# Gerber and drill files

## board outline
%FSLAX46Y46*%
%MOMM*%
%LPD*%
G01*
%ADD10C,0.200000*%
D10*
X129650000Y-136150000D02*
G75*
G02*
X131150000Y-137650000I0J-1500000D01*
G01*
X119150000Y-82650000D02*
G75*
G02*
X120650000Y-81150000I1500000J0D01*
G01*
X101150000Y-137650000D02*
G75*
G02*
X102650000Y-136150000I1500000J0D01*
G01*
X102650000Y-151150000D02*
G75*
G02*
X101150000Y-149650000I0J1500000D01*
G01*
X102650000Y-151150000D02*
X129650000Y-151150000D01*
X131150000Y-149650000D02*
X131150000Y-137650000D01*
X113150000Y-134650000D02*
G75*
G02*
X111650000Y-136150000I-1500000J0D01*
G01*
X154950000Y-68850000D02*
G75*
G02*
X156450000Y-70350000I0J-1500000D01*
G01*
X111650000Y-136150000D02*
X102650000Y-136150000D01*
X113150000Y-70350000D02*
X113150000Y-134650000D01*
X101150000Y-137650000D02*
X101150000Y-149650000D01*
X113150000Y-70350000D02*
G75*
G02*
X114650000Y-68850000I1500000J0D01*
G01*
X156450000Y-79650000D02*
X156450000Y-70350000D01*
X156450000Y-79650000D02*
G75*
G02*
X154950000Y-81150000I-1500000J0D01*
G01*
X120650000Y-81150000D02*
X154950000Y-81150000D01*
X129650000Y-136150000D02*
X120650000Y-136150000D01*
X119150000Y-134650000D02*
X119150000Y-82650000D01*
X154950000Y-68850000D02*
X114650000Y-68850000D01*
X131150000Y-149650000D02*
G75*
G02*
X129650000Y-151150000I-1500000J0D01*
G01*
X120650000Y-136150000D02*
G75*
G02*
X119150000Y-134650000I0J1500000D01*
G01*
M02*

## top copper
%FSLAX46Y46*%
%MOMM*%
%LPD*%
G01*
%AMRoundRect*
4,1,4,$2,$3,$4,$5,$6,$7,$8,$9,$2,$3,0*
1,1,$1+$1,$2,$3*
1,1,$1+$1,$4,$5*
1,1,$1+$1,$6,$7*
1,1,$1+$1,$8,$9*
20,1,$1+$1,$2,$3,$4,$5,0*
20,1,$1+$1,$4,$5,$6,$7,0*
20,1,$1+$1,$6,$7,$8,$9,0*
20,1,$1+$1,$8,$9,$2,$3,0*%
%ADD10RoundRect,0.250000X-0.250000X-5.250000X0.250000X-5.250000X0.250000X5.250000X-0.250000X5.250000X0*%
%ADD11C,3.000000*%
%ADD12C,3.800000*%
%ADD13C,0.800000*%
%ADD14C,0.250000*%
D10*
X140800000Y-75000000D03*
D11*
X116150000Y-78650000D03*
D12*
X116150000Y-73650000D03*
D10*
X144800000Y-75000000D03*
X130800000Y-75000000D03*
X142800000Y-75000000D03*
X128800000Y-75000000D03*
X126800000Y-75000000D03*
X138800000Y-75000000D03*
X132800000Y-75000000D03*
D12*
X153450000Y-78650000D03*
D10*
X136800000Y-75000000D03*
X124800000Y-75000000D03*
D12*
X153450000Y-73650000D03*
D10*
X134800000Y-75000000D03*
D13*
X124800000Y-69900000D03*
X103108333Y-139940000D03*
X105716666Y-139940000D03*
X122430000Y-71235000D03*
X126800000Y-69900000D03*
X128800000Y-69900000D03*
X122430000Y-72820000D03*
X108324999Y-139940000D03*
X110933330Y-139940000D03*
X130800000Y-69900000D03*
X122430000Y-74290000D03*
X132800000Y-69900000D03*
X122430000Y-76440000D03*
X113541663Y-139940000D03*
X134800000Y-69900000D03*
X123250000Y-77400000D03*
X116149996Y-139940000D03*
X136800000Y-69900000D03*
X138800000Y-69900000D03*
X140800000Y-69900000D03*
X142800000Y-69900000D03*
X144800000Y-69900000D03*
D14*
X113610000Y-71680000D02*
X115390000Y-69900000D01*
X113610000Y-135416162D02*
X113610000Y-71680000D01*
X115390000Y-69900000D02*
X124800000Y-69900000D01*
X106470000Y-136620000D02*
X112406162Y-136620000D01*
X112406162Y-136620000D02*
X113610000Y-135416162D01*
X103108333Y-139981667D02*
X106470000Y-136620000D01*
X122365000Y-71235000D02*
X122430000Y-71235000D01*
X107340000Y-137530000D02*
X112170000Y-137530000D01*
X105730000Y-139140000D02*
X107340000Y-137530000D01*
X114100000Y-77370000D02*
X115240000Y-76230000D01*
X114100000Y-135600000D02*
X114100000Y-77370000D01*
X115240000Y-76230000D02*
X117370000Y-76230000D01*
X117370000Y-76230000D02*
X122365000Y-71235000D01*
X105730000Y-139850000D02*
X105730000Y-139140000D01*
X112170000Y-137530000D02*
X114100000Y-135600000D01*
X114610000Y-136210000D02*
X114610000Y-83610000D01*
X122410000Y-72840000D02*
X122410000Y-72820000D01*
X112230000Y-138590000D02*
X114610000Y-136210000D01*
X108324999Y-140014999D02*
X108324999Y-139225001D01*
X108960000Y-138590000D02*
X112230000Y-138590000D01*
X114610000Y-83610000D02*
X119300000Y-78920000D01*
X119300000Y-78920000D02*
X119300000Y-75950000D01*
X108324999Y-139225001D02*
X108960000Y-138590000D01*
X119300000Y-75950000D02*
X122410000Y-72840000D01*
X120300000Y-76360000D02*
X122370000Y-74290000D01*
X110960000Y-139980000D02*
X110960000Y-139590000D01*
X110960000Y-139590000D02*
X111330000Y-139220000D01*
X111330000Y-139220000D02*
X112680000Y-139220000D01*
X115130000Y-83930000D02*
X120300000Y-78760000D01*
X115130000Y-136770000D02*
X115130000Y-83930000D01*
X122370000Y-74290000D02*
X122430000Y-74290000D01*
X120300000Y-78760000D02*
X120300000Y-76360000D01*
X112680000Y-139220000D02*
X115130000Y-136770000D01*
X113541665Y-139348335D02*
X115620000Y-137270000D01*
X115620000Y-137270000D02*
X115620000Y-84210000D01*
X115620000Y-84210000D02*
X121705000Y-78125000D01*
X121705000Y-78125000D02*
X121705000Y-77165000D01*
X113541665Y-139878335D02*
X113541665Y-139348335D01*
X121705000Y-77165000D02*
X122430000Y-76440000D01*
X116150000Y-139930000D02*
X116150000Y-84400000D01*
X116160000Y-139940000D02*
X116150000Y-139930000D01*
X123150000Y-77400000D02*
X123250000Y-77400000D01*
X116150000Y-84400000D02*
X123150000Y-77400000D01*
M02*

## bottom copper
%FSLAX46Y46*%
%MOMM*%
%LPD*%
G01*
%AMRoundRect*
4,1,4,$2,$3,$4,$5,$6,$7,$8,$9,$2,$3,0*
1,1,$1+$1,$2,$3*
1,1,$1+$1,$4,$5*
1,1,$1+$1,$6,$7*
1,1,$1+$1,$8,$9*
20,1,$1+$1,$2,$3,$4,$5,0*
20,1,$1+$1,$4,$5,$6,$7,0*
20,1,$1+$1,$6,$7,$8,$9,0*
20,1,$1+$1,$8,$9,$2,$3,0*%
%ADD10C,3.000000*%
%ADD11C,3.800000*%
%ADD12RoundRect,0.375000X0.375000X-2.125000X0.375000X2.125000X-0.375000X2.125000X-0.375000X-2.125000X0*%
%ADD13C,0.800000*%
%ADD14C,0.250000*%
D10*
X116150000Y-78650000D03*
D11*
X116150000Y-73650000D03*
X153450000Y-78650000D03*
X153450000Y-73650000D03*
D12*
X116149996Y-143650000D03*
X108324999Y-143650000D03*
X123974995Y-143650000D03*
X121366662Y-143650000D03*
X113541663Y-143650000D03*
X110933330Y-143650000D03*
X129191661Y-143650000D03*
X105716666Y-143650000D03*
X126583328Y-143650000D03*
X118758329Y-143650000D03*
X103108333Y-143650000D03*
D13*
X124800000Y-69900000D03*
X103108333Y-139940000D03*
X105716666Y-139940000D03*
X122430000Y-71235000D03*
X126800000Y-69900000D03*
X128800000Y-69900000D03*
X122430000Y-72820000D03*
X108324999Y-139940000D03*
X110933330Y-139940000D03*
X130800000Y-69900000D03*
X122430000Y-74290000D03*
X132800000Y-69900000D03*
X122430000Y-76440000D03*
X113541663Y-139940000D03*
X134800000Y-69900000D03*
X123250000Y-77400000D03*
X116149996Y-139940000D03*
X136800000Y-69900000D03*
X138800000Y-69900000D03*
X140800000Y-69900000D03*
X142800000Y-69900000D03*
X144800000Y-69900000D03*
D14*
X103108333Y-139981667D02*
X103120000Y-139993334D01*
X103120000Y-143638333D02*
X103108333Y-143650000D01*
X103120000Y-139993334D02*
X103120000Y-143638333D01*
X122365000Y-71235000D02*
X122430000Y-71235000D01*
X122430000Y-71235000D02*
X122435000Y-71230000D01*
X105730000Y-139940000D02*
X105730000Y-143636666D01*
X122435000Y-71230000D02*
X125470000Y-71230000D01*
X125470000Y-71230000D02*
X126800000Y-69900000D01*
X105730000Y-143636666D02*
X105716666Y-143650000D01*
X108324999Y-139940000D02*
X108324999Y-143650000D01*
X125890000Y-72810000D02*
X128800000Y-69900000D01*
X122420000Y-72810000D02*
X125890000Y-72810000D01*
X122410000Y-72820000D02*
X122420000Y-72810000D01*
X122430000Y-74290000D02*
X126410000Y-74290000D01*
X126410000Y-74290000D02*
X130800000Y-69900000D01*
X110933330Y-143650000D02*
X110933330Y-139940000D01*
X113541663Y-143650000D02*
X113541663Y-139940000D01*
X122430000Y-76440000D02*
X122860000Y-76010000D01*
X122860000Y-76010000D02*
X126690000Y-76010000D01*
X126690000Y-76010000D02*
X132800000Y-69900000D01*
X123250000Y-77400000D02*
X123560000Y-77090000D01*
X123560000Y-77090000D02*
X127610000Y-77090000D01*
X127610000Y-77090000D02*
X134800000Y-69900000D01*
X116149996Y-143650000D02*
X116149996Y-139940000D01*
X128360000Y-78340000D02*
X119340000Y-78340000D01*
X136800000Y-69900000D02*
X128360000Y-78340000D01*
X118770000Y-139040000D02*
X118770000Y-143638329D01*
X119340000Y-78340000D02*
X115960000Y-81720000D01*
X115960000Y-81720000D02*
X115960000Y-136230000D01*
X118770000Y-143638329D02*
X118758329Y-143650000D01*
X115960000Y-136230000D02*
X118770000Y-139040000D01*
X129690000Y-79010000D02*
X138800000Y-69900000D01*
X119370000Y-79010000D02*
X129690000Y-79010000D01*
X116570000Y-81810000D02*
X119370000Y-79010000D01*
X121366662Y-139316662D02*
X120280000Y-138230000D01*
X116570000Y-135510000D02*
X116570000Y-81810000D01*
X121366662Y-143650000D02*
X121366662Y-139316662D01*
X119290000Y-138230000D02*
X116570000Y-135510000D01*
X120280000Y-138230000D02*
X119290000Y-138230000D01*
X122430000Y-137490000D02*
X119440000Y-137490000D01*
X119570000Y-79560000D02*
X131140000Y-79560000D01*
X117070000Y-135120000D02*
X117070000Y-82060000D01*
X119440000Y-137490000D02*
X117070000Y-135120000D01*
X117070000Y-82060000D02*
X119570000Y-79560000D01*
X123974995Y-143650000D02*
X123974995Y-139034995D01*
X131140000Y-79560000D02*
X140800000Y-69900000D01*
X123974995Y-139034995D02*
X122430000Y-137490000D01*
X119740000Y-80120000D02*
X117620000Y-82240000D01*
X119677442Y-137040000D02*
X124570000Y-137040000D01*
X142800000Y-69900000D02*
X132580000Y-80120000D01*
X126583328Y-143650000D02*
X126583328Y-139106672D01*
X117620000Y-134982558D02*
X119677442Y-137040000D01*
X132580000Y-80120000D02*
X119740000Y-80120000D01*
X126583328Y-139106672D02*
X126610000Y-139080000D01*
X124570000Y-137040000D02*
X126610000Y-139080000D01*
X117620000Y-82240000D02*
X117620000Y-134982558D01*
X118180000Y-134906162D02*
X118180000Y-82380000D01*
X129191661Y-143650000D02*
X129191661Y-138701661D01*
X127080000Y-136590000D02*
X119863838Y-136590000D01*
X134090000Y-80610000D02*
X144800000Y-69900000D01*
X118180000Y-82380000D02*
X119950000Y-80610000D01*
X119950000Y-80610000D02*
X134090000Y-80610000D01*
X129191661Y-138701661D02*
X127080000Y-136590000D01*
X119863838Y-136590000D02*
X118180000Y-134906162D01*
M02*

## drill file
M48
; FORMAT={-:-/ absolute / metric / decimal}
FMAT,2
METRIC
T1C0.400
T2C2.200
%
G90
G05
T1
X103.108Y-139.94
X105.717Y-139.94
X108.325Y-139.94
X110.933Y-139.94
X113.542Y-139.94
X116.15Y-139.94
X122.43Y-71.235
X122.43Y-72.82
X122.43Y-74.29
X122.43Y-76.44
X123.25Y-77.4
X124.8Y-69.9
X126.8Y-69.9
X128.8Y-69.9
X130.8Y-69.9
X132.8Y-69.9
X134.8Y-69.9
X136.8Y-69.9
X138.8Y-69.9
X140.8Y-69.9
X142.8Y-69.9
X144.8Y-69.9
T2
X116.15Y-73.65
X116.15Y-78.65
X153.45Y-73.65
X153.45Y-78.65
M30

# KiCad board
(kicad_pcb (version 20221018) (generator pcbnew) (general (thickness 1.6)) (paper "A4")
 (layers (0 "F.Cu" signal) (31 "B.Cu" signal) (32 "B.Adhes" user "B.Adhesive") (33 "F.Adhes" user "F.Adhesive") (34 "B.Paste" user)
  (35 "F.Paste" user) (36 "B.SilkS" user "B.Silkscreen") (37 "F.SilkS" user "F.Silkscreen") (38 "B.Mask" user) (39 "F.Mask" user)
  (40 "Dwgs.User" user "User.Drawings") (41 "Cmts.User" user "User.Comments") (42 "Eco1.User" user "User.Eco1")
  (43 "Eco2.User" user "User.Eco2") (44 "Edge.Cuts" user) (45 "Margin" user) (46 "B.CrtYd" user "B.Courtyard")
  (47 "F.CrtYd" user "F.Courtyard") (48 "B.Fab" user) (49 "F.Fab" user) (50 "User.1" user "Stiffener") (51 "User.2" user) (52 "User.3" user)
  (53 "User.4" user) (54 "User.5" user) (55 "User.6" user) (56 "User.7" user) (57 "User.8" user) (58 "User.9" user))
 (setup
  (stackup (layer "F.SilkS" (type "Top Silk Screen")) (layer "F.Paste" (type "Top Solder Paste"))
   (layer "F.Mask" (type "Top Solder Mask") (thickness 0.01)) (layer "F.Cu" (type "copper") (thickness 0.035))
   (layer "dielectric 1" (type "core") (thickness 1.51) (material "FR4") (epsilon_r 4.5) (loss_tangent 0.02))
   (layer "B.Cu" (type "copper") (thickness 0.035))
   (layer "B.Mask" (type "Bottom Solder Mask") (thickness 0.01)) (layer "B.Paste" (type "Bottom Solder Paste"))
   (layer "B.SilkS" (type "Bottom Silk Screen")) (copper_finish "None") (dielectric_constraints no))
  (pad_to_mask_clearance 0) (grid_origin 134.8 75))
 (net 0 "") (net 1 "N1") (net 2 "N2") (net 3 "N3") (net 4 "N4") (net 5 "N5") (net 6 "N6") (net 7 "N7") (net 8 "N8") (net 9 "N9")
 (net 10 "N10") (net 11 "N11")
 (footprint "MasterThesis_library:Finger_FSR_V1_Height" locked (layer "F.Cu") (at 140.8 75)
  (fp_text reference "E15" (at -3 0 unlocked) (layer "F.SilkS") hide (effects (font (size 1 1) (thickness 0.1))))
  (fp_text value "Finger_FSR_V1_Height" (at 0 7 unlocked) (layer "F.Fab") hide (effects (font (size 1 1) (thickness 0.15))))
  (pad "1" smd roundrect locked (at 0 0) (size 1 11) (layers "F.Cu" "F.Paste" "F.Mask") (roundrect_rratio 0.25) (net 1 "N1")
   (thermal_bridge_angle 45)))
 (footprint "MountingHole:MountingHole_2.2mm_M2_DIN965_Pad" (layer "F.Cu") (at 116.15 78.65)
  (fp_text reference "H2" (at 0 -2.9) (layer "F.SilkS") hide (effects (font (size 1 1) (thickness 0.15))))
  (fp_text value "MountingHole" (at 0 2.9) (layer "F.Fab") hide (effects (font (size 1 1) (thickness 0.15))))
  (pad "1" thru_hole circle (at 0 0) (size 3 3) (drill 2.2) (layers "*.Cu" "*.Mask")))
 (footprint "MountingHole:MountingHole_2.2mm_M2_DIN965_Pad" (layer "F.Cu") (at 116.15 73.65)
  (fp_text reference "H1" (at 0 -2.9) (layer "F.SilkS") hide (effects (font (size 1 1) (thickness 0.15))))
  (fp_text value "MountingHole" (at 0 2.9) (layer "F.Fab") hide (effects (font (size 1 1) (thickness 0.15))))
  (pad "1" thru_hole circle (at 0 0) (size 3.8 3.8) (drill 2.2) (layers "*.Cu" "*.Mask")))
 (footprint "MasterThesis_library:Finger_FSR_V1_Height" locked (layer "F.Cu") (at 144.8 75)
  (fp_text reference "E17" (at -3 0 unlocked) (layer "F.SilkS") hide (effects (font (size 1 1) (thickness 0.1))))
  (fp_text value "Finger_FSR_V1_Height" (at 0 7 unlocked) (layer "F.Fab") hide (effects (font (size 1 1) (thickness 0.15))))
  (pad "1" smd roundrect locked (at 0 0) (size 1 11) (layers "F.Cu" "F.Paste" "F.Mask") (roundrect_rratio 0.25) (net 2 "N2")
   (thermal_bridge_angle 45)))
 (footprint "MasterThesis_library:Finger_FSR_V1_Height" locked (layer "F.Cu") (at 130.8 75)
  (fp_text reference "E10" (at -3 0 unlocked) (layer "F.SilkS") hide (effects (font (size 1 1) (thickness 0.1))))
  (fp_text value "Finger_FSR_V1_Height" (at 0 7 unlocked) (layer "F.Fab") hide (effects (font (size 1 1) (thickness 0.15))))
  (pad "1" smd roundrect locked (at 0 0) (size 1 11) (layers "F.Cu" "F.Paste" "F.Mask") (roundrect_rratio 0.25) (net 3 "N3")
   (thermal_bridge_angle 45)))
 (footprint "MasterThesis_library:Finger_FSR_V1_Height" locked (layer "F.Cu") (at 142.8 75)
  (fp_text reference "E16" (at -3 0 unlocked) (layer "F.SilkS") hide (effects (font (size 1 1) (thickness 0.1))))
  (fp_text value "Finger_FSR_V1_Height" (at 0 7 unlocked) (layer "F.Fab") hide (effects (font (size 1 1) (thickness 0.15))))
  (pad "1" smd roundrect locked (at 0 0) (size 1 11) (layers "F.Cu" "F.Paste" "F.Mask") (roundrect_rratio 0.25) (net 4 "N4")
   (thermal_bridge_angle 45)))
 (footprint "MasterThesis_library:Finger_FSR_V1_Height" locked (layer "F.Cu") (at 128.8 75)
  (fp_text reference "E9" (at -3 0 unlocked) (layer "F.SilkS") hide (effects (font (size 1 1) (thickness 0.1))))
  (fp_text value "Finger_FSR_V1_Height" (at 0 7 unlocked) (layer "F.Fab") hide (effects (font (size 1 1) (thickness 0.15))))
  (pad "1" smd roundrect locked (at 0 0) (size 1 11) (layers "F.Cu" "F.Paste" "F.Mask") (roundrect_rratio 0.25) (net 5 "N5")
   (thermal_bridge_angle 45)))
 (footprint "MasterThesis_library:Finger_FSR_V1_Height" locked (layer "F.Cu") (at 126.8 75)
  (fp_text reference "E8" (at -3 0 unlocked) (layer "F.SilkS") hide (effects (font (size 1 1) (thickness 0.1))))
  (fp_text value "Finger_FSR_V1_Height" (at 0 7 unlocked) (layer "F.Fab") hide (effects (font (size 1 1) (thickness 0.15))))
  (pad "1" smd roundrect locked (at 0 0) (size 1 11) (layers "F.Cu" "F.Paste" "F.Mask") (roundrect_rratio 0.25) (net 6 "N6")
   (thermal_bridge_angle 45)))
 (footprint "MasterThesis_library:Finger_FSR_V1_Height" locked (layer "F.Cu") (at 138.8 75)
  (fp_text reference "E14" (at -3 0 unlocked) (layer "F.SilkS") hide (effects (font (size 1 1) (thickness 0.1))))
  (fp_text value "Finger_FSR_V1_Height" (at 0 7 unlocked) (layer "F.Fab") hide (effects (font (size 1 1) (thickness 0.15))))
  (pad "1" smd roundrect locked (at 0 0) (size 1 11) (layers "F.Cu" "F.Paste" "F.Mask") (roundrect_rratio 0.25) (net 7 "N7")
   (thermal_bridge_angle 45)))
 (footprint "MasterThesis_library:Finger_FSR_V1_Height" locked (layer "F.Cu") (at 132.8 75)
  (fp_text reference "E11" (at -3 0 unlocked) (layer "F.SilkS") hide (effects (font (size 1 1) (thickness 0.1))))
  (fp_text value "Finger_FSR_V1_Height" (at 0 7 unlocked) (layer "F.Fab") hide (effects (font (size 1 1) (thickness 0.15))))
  (pad "1" smd roundrect locked (at 0 0) (size 1 11) (layers "F.Cu" "F.Paste" "F.Mask") (roundrect_rratio 0.25) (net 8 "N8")
   (thermal_bridge_angle 45)))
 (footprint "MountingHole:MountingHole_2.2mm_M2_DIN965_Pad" (layer "F.Cu") (at 153.45 78.65)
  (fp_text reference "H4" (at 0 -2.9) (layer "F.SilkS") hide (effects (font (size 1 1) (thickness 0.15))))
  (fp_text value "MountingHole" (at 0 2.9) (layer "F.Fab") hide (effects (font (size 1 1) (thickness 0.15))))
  (pad "1" thru_hole circle (at 0 0) (size 3.8 3.8) (drill 2.2) (layers "*.Cu" "*.Mask")))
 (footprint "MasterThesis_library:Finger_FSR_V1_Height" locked (layer "F.Cu") (at 136.8 75)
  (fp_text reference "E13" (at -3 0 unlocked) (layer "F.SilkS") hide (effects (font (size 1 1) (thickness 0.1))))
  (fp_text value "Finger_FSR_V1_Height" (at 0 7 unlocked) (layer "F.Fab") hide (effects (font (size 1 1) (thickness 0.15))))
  (pad "1" smd roundrect locked (at 0 0) (size 1 11) (layers "F.Cu" "F.Paste" "F.Mask") (roundrect_rratio 0.25) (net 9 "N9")
   (thermal_bridge_angle 45)))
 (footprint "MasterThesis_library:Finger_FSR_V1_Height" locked (layer "F.Cu") (at 124.8 75)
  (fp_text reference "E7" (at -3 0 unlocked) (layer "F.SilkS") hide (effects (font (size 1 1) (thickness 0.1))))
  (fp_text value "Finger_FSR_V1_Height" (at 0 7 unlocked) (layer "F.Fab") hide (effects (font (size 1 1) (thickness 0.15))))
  (pad "1" smd roundrect locked (at 0 0) (size 1 11) (layers "F.Cu" "F.Paste" "F.Mask") (roundrect_rratio 0.25) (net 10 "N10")
   (thermal_bridge_angle 45)))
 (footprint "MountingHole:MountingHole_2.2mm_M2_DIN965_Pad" (layer "F.Cu") (at 153.45 73.65)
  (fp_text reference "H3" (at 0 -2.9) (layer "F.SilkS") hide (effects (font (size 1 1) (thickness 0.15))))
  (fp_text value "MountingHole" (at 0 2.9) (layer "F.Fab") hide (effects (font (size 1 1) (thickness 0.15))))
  (pad "1" thru_hole circle (at 0 0) (size 3.8 3.8) (drill 2.2) (layers "*.Cu" "*.Mask")))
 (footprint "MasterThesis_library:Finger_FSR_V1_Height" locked (layer "F.Cu") (at 134.8 75)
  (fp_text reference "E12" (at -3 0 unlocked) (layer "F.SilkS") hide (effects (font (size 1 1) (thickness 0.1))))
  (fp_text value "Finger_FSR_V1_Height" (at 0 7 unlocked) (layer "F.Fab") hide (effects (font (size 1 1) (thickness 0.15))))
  (pad "1" smd roundrect locked (at 0 0) (size 1 11) (layers "F.Cu" "F.Paste" "F.Mask") (roundrect_rratio 0.25) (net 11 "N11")
   (thermal_bridge_angle 45)))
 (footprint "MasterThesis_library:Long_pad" (layer "B.Cu") (at 116.149996 143.65 90)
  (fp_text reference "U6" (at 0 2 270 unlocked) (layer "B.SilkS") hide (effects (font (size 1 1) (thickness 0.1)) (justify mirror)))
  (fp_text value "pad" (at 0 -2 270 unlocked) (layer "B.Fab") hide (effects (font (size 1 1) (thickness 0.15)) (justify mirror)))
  (pad "1" smd roundrect (at 0 0 90) (size 5 1.5) (layers "B.Cu" "B.Paste" "B.Mask") (roundrect_rratio 0.25) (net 11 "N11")
   (thermal_bridge_angle 45)))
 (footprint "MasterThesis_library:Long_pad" (layer "B.Cu") (at 108.324999 143.65 90)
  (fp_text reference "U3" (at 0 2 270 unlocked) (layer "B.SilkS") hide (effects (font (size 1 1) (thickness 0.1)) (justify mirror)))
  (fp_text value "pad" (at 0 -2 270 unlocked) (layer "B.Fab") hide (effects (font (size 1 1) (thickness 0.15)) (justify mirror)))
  (pad "1" smd roundrect (at 0 0 90) (size 5 1.5) (layers "B.Cu" "B.Paste" "B.Mask") (roundrect_rratio 0.25) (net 5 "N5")
   (thermal_bridge_angle 45)))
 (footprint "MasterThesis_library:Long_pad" (layer "B.Cu") (at 123.974995 143.65 90)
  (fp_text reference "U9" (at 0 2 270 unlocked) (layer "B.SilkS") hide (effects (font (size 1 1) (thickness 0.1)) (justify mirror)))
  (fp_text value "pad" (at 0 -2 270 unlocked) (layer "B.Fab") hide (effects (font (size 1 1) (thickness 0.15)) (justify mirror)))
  (pad "1" smd roundrect (at 0 0 90) (size 5 1.5) (layers "B.Cu" "B.Paste" "B.Mask") (roundrect_rratio 0.25) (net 1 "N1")
   (thermal_bridge_angle 45)))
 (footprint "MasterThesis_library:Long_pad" (layer "B.Cu") (at 121.366662 143.65 90)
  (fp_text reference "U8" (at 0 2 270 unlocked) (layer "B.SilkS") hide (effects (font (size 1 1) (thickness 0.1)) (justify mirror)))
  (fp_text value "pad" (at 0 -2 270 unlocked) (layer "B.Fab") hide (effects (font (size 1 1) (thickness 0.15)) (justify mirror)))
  (pad "1" smd roundrect (at 0 0 90) (size 5 1.5) (layers "B.Cu" "B.Paste" "B.Mask") (roundrect_rratio 0.25) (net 7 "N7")
   (thermal_bridge_angle 45)))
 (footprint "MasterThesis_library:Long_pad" (layer "B.Cu") (at 113.541663 143.65 90)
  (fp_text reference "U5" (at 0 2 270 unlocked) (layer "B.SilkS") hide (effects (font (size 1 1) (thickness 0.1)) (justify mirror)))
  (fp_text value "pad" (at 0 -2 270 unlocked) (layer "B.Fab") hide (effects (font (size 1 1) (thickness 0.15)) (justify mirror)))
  (pad "1" smd roundrect (at 0 0 90) (size 5 1.5) (layers "B.Cu" "B.Paste" "B.Mask") (roundrect_rratio 0.25) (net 8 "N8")
   (thermal_bridge_angle 45)))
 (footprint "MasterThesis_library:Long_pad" (layer "B.Cu") (at 110.93333 143.65 90)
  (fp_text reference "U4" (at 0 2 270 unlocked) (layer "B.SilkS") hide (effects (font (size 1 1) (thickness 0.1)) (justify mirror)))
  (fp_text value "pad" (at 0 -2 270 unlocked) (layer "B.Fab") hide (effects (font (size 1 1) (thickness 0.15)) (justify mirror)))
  (pad "1" smd roundrect (at 0 0 90) (size 5 1.5) (layers "B.Cu" "B.Paste" "B.Mask") (roundrect_rratio 0.25) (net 3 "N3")
   (thermal_bridge_angle 45)))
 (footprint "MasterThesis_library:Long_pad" (layer "B.Cu") (at 129.191661 143.65 90)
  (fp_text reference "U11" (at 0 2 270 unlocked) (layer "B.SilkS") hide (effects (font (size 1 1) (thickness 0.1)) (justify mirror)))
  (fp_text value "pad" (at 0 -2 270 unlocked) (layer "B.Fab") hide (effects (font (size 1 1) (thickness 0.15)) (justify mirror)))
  (pad "1" smd roundrect (at 0 0 90) (size 5 1.5) (layers "B.Cu" "B.Paste" "B.Mask") (roundrect_rratio 0.25) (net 2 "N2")
   (thermal_bridge_angle 45)))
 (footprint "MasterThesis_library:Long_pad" (layer "B.Cu") (at 105.716666 143.65 90)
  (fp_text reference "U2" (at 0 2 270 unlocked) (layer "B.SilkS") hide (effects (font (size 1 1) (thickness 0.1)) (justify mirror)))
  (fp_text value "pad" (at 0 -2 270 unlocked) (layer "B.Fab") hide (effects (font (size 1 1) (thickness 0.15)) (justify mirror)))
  (pad "1" smd roundrect (at 0 0 90) (size 5 1.5) (layers "B.Cu" "B.Paste" "B.Mask") (roundrect_rratio 0.25) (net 6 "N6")
   (thermal_bridge_angle 45)))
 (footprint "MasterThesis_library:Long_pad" (layer "B.Cu") (at 126.583328 143.65 90)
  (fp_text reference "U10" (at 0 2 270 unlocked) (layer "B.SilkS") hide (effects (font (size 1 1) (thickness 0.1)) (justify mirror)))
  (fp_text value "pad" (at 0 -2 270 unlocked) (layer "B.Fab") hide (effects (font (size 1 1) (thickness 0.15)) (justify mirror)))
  (pad "1" smd roundrect (at 0 0 90) (size 5 1.5) (layers "B.Cu" "B.Paste" "B.Mask") (roundrect_rratio 0.25) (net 4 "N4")
   (thermal_bridge_angle 45)))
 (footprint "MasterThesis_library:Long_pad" (layer "B.Cu") (at 118.758329 143.65 90)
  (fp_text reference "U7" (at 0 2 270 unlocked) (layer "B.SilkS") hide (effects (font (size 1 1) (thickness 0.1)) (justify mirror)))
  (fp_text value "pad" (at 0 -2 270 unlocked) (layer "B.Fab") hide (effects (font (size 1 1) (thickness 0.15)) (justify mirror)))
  (pad "1" smd roundrect (at 0 0 90) (size 5 1.5) (layers "B.Cu" "B.Paste" "B.Mask") (roundrect_rratio 0.25) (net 9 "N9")
   (thermal_bridge_angle 45)))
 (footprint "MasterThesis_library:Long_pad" (layer "B.Cu") (at 103.108333 143.65 90)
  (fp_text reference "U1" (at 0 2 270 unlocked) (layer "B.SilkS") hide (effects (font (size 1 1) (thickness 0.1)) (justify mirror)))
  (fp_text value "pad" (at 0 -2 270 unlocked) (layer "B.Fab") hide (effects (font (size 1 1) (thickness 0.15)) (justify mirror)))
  (pad "1" smd roundrect (at 0 0 90) (size 5 1.5) (layers "B.Cu" "B.Paste" "B.Mask") (roundrect_rratio 0.25) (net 10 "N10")
   (thermal_bridge_angle 45)))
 (gr_arc locked (start 129.65 136.15) (mid 130.71066 136.58934) (end 131.15 137.65) (stroke (width 0.2) (type solid)) (layer "Edge.Cuts"))
 (gr_arc locked (start 119.15 82.65) (mid 119.58934 81.58934) (end 120.65 81.15) (stroke (width 0.2) (type solid)) (layer "Edge.Cuts"))
 (gr_arc locked (start 101.15 137.65) (mid 101.58934 136.58934) (end 102.65 136.15) (stroke (width 0.2) (type solid)) (layer "Edge.Cuts"))
 (gr_arc locked (start 102.65 151.15) (mid 101.58934 150.71066) (end 101.15 149.65) (stroke (width 0.2) (type solid)) (layer "Edge.Cuts"))
 (gr_line locked (start 102.65 151.15) (end 129.65 151.15) (stroke (width 0.2) (type solid)) (layer "Edge.Cuts"))
 (gr_line locked (start 131.15 149.65) (end 131.15 137.65) (stroke (width 0.2) (type solid)) (layer "Edge.Cuts"))
 (gr_arc locked (start 113.15 134.65) (mid 112.71066 135.71066) (end 111.65 136.15) (stroke (width 0.2) (type solid)) (layer "Edge.Cuts"))
 (gr_arc locked (start 154.95 68.85) (mid 156.01066 69.28934) (end 156.45 70.35) (stroke (width 0.2) (type solid)) (layer "Edge.Cuts"))
 (gr_line locked (start 111.65 136.15) (end 102.65 136.15) (stroke (width 0.2) (type solid)) (layer "Edge.Cuts"))
 (gr_line locked (start 113.15 70.35) (end 113.15 134.65) (stroke (width 0.2) (type solid)) (layer "Edge.Cuts"))
 (gr_line locked (start 101.15 137.65) (end 101.15 149.65) (stroke (width 0.2) (type solid)) (layer "Edge.Cuts"))
 (gr_arc locked (start 113.15 70.35) (mid 113.58934 69.28934) (end 114.65 68.85) (stroke (width 0.2) (type solid)) (layer "Edge.Cuts"))
 (gr_line locked (start 156.45 79.65) (end 156.45 70.35) (stroke (width 0.2) (type solid)) (layer "Edge.Cuts"))
 (gr_arc locked (start 156.45 79.65) (mid 156.01066 80.71066) (end 154.95 81.15) (stroke (width 0.2) (type solid)) (layer "Edge.Cuts"))
 (gr_line locked (start 120.65 81.15) (end 154.95 81.15) (stroke (width 0.2) (type solid)) (layer "Edge.Cuts"))
 (gr_line locked (start 129.65 136.15) (end 120.65 136.15) (stroke (width 0.2) (type solid)) (layer "Edge.Cuts"))
 (gr_line locked (start 119.15 134.65) (end 119.15 82.65) (stroke (width 0.2) (type solid)) (layer "Edge.Cuts"))
 (gr_line locked (start 154.95 68.85) (end 114.65 68.85) (stroke (width 0.2) (type solid)) (layer "Edge.Cuts"))
 (gr_arc locked (start 131.15 149.65) (mid 130.71066 150.71066) (end 129.65 151.15) (stroke (width 0.2) (type solid)) (layer "Edge.Cuts"))
 (gr_arc locked (start 120.65 136.15) (mid 119.58934 135.71066) (end 119.15 134.65) (stroke (width 0.2) (type solid)) (layer "Edge.Cuts"))
 (segment (start 113.61 71.68) (end 115.39 69.9) (width 0.25) (layer "F.Cu") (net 10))
 (segment (start 113.61 135.416162) (end 113.61 71.68) (width 0.25) (layer "F.Cu") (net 10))
 (segment (start 115.39 69.9) (end 124.8 69.9) (width 0.25) (layer "F.Cu") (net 10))
 (segment (start 106.47 136.62) (end 112.406162 136.62) (width 0.25) (layer "F.Cu") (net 10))
 (segment (start 112.406162 136.62) (end 113.61 135.416162) (width 0.25) (layer "F.Cu") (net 10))
 (segment (start 103.108333 139.981667) (end 106.47 136.62) (width 0.25) (layer "F.Cu") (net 10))
 (via (at 124.8 69.9) (size 0.8) (drill 0.4) (layers "F.Cu" "B.Cu") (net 10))
 (via (at 103.108333 139.94) (size 0.8) (drill 0.4) (layers "F.Cu" "B.Cu") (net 10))
 (segment (start 103.108333 139.981667) (end 103.12 139.993334) (width 0.25) (layer "B.Cu") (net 10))
 (segment (start 103.12 143.638333) (end 103.108333 143.65) (width 0.25) (layer "B.Cu") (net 10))
 (segment (start 103.12 139.993334) (end 103.12 143.638333) (width 0.25) (layer "B.Cu") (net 10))
 (segment (start 122.365 71.235) (end 122.43 71.235) (width 0.25) (layer "F.Cu") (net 6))
 (segment (start 107.34 137.53) (end 112.17 137.53) (width 0.25) (layer "F.Cu") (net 6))
 (segment (start 105.73 139.14) (end 107.34 137.53) (width 0.25) (layer "F.Cu") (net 6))
 (segment (start 114.1 77.37) (end 115.24 76.23) (width 0.25) (layer "F.Cu") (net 6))
 (segment (start 114.1 135.6) (end 114.1 77.37) (width 0.25) (layer "F.Cu") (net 6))
 (segment (start 115.24 76.23) (end 117.37 76.23) (width 0.25) (layer "F.Cu") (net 6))
 (segment (start 117.37 76.23) (end 122.365 71.235) (width 0.25) (layer "F.Cu") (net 6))
 (segment (start 105.73 139.85) (end 105.73 139.14) (width 0.25) (layer "F.Cu") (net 6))
 (segment (start 112.17 137.53) (end 114.1 135.6) (width 0.25) (layer "F.Cu") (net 6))
 (via (at 105.716666 139.94) (size 0.8) (drill 0.4) (layers "F.Cu" "B.Cu") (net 6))
 (via (at 122.43 71.235) (size 0.8) (drill 0.4) (layers "F.Cu" "B.Cu") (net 6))
 (via (at 126.8 69.9) (size 0.8) (drill 0.4) (layers "F.Cu" "B.Cu") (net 6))
 (segment (start 122.365 71.235) (end 122.43 71.235) (width 0.25) (layer "B.Cu") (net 6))
 (segment (start 122.43 71.235) (end 122.435 71.23) (width 0.25) (layer "B.Cu") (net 6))
 (segment (start 105.73 139.94) (end 105.73 143.636666) (width 0.25) (layer "B.Cu") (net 6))
 (segment (start 122.435 71.23) (end 125.47 71.23) (width 0.25) (layer "B.Cu") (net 6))
 (segment (start 125.47 71.23) (end 126.8 69.9) (width 0.25) (layer "B.Cu") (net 6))
 (segment (start 105.73 143.636666) (end 105.716666 143.65) (width 0.25) (layer "B.Cu") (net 6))
 (segment (start 114.61 136.21) (end 114.61 83.61) (width 0.25) (layer "F.Cu") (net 5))
 (segment (start 122.41 72.84) (end 122.41 72.82) (width 0.25) (layer "F.Cu") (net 5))
 (segment (start 112.23 138.59) (end 114.61 136.21) (width 0.25) (layer "F.Cu") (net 5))
 (segment (start 108.324999 140.014999) (end 108.324999 139.225001) (width 0.25) (layer "F.Cu") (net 5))
 (segment (start 108.96 138.59) (end 112.23 138.59) (width 0.25) (layer "F.Cu") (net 5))
 (segment (start 114.61 83.61) (end 119.3 78.92) (width 0.25) (layer "F.Cu") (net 5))
 (segment (start 119.3 78.92) (end 119.3 75.95) (width 0.25) (layer "F.Cu") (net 5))
 (segment (start 108.324999 139.225001) (end 108.96 138.59) (width 0.25) (layer "F.Cu") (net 5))
 (segment (start 119.3 75.95) (end 122.41 72.84) (width 0.25) (layer "F.Cu") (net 5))
 (via (at 128.8 69.9) (size 0.8) (drill 0.4) (layers "F.Cu" "B.Cu") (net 5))
 (via (at 122.43 72.82) (size 0.8) (drill 0.4) (layers "F.Cu" "B.Cu") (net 5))
 (via (at 108.324999 139.94) (size 0.8) (drill 0.4) (layers "F.Cu" "B.Cu") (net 5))
 (segment (start 108.324999 139.94) (end 108.324999 143.65) (width 0.25) (layer "B.Cu") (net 5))
 (segment (start 125.89 72.81) (end 128.8 69.9) (width 0.25) (layer "B.Cu") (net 5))
 (segment (start 122.42 72.81) (end 125.89 72.81) (width 0.25) (layer "B.Cu") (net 5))
 (segment (start 122.41 72.82) (end 122.42 72.81) (width 0.25) (layer "B.Cu") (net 5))
 (segment (start 120.3 76.36) (end 122.37 74.29) (width 0.25) (layer "F.Cu") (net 3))
 (segment (start 110.96 139.98) (end 110.96 139.59) (width 0.25) (layer "F.Cu") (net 3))
 (segment (start 110.96 139.59) (end 111.33 139.22) (width 0.25) (layer "F.Cu") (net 3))
 (segment (start 111.33 139.22) (end 112.68 139.22) (width 0.25) (layer "F.Cu") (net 3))
 (segment (start 115.13 83.93) (end 120.3 78.76) (width 0.25) (layer "F.Cu") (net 3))
 (segment (start 115.13 136.77) (end 115.13 83.93) (width 0.25) (layer "F.Cu") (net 3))
 (segment (start 122.37 74.29) (end 122.43 74.29) (width 0.25) (layer "F.Cu") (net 3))
 (segment (start 120.3 78.76) (end 120.3 76.36) (width 0.25) (layer "F.Cu") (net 3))
 (segment (start 112.68 139.22) (end 115.13 136.77) (width 0.25) (layer "F.Cu") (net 3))
 (via (at 110.93333 139.94) (size 0.8) (drill 0.4) (layers "F.Cu" "B.Cu") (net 3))
 (via (at 130.8 69.9) (size 0.8) (drill 0.4) (layers "F.Cu" "B.Cu") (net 3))
 (via (at 122.43 74.29) (size 0.8) (drill 0.4) (layers "F.Cu" "B.Cu") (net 3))
 (segment (start 122.43 74.29) (end 126.41 74.29) (width 0.25) (layer "B.Cu") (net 3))
 (segment (start 126.41 74.29) (end 130.8 69.9) (width 0.25) (layer "B.Cu") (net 3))
 (segment (start 110.93333 143.65) (end 110.93333 139.94) (width 0.25) (layer "B.Cu") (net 3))
 (segment (start 113.541665 139.348335) (end 115.62 137.27) (width 0.25) (layer "F.Cu") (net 8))
 (segment (start 115.62 137.27) (end 115.62 84.21) (width 0.25) (layer "F.Cu") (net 8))
 (segment (start 115.62 84.21) (end 121.705 78.125) (width 0.25) (layer "F.Cu") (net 8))
 (segment (start 121.705 78.125) (end 121.705 77.165) (width 0.25) (layer "F.Cu") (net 8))
 (segment (start 113.541665 139.878335) (end 113.541665 139.348335) (width 0.25) (layer "F.Cu") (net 8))
 (segment (start 121.705 77.165) (end 122.43 76.44) (width 0.25) (layer "F.Cu") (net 8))
 (via (at 132.8 69.9) (size 0.8) (drill 0.4) (layers "F.Cu" "B.Cu") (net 8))
 (via (at 122.43 76.44) (size 0.8) (drill 0.4) (layers "F.Cu" "B.Cu") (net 8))
 (via (at 113.541663 139.94) (size 0.8) (drill 0.4) (layers "F.Cu" "B.Cu") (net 8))
 (segment (start 113.541663 143.65) (end 113.541663 139.94) (width 0.25) (layer "B.Cu") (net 8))
 (segment (start 122.43 76.44) (end 122.86 76.01) (width 0.25) (layer "B.Cu") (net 8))
 (segment (start 122.86 76.01) (end 126.69 76.01) (width 0.25) (layer "B.Cu") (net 8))
 (segment (start 126.69 76.01) (end 132.8 69.9) (width 0.25) (layer "B.Cu") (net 8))
 (segment (start 116.15 139.93) (end 116.15 84.4) (width 0.25) (layer "F.Cu") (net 11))
 (segment (start 116.16 139.94) (end 116.15 139.93) (width 0.25) (layer "F.Cu") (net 11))
 (segment (start 123.15 77.4) (end 123.25 77.4) (width 0.25) (layer "F.Cu") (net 11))
 (segment (start 116.15 84.4) (end 123.15 77.4) (width 0.25) (layer "F.Cu") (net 11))
 (via (at 134.8 69.9) (size 0.8) (drill 0.4) (layers "F.Cu" "B.Cu") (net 11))
 (via (at 123.25 77.4) (size 0.8) (drill 0.4) (layers "F.Cu" "B.Cu") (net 11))
 (via (at 116.149996 139.94) (size 0.8) (drill 0.4) (layers "F.Cu" "B.Cu") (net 11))
 (segment (start 123.25 77.4) (end 123.56 77.09) (width 0.25) (layer "B.Cu") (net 11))
 (segment (start 123.56 77.09) (end 127.61 77.09) (width 0.25) (layer "B.Cu") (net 11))
 (segment (start 127.61 77.09) (end 134.8 69.9) (width 0.25) (layer "B.Cu") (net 11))
 (segment (start 116.149996 143.65) (end 116.149996 139.94) (width 0.25) (layer "B.Cu") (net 11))
 (via (at 136.8 69.9) (size 0.8) (drill 0.4) (layers "F.Cu" "B.Cu") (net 9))
 (segment (start 128.36 78.34) (end 119.34 78.34) (width 0.25) (layer "B.Cu") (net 9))
 (segment (start 136.8 69.9) (end 128.36 78.34) (width 0.25) (layer "B.Cu") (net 9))
 (segment (start 118.77 139.04) (end 118.77 143.638329) (width 0.25) (layer "B.Cu") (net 9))
 (segment (start 119.34 78.34) (end 115.96 81.72) (width 0.25) (layer "B.Cu") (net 9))
 (segment (start 115.96 81.72) (end 115.96 136.23) (width 0.25) (layer "B.Cu") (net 9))
 (segment (start 118.77 143.638329) (end 118.758329 143.65) (width 0.25) (layer "B.Cu") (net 9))
 (segment (start 115.96 136.23) (end 118.77 139.04) (width 0.25) (layer "B.Cu") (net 9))
 (via (at 138.8 69.9) (size 0.8) (drill 0.4) (layers "F.Cu" "B.Cu") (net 7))
 (segment (start 129.69 79.01) (end 138.8 69.9) (width 0.25) (layer "B.Cu") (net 7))
 (segment (start 119.37 79.01) (end 129.69 79.01) (width 0.25) (layer "B.Cu") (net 7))
 (segment (start 116.57 81.81) (end 119.37 79.01) (width 0.25) (layer "B.Cu") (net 7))
 (segment (start 121.366662 139.316662) (end 120.28 138.23) (width 0.25) (layer "B.Cu") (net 7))
 (segment (start 116.57 135.51) (end 116.57 81.81) (width 0.25) (layer "B.Cu") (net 7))
 (segment (start 121.366662 143.65) (end 121.366662 139.316662) (width 0.25) (layer "B.Cu") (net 7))
 (segment (start 119.29 138.23) (end 116.57 135.51) (width 0.25) (layer "B.Cu") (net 7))
 (segment (start 120.28 138.23) (end 119.29 138.23) (width 0.25) (layer "B.Cu") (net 7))
 (via (at 140.8 69.9) (size 0.8) (drill 0.4) (layers "F.Cu" "B.Cu") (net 1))
 (segment (start 122.43 137.49) (end 119.44 137.49) (width 0.25) (layer "B.Cu") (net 1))
 (segment (start 119.57 79.56) (end 131.14 79.56) (width 0.25) (layer "B.Cu") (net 1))
 (segment (start 117.07 135.12) (end 117.07 82.06) (width 0.25) (layer "B.Cu") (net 1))
 (segment (start 119.44 137.49) (end 117.07 135.12) (width 0.25) (layer "B.Cu") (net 1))
 (segment (start 117.07 82.06) (end 119.57 79.56) (width 0.25) (layer "B.Cu") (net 1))
 (segment (start 123.974995 143.65) (end 123.974995 139.034995) (width 0.25) (layer "B.Cu") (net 1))
 (segment (start 131.14 79.56) (end 140.8 69.9) (width 0.25) (layer "B.Cu") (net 1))
 (segment (start 123.974995 139.034995) (end 122.43 137.49) (width 0.25) (layer "B.Cu") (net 1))
 (via (at 142.8 69.9) (size 0.8) (drill 0.4) (layers "F.Cu" "B.Cu") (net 4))
 (segment (start 119.74 80.12) (end 117.62 82.24) (width 0.25) (layer "B.Cu") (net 4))
 (segment (start 119.677442 137.04) (end 124.57 137.04) (width 0.25) (layer "B.Cu") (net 4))
 (segment (start 142.8 69.9) (end 132.58 80.12) (width 0.25) (layer "B.Cu") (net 4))
 (segment (start 126.583328 143.65) (end 126.583328 139.106672) (width 0.25) (layer "B.Cu") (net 4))
 (segment (start 117.62 134.982558) (end 119.677442 137.04) (width 0.25) (layer "B.Cu") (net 4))
 (segment (start 132.58 80.12) (end 119.74 80.12) (width 0.25) (layer "B.Cu") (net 4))
 (segment (start 126.583328 139.106672) (end 126.61 139.08) (width 0.25) (layer "B.Cu") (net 4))
 (segment (start 124.57 137.04) (end 126.61 139.08) (width 0.25) (layer "B.Cu") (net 4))
 (segment (start 117.62 82.24) (end 117.62 134.982558) (width 0.25) (layer "B.Cu") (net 4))
 (via (at 144.8 69.9) (size 0.8) (drill 0.4) (layers "F.Cu" "B.Cu") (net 2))
 (segment (start 118.18 134.906162) (end 118.18 82.38) (width 0.25) (layer "B.Cu") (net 2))
 (segment (start 129.191661 143.65) (end 129.191661 138.701661) (width 0.25) (layer "B.Cu") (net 2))
 (segment (start 127.08 136.59) (end 119.863838 136.59) (width 0.25) (layer "B.Cu") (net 2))
 (segment (start 134.09 80.61) (end 144.8 69.9) (width 0.25) (layer "B.Cu") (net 2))
 (segment (start 118.18 82.38) (end 119.95 80.61) (width 0.25) (layer "B.Cu") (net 2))
 (segment (start 119.95 80.61) (end 134.09 80.61) (width 0.25) (layer "B.Cu") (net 2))
 (segment (start 129.191661 138.701661) (end 127.08 136.59) (width 0.25) (layer "B.Cu") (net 2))
 (segment (start 119.863838 136.59) (end 118.18 134.906162) (width 0.25) (layer "B.Cu") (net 2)))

